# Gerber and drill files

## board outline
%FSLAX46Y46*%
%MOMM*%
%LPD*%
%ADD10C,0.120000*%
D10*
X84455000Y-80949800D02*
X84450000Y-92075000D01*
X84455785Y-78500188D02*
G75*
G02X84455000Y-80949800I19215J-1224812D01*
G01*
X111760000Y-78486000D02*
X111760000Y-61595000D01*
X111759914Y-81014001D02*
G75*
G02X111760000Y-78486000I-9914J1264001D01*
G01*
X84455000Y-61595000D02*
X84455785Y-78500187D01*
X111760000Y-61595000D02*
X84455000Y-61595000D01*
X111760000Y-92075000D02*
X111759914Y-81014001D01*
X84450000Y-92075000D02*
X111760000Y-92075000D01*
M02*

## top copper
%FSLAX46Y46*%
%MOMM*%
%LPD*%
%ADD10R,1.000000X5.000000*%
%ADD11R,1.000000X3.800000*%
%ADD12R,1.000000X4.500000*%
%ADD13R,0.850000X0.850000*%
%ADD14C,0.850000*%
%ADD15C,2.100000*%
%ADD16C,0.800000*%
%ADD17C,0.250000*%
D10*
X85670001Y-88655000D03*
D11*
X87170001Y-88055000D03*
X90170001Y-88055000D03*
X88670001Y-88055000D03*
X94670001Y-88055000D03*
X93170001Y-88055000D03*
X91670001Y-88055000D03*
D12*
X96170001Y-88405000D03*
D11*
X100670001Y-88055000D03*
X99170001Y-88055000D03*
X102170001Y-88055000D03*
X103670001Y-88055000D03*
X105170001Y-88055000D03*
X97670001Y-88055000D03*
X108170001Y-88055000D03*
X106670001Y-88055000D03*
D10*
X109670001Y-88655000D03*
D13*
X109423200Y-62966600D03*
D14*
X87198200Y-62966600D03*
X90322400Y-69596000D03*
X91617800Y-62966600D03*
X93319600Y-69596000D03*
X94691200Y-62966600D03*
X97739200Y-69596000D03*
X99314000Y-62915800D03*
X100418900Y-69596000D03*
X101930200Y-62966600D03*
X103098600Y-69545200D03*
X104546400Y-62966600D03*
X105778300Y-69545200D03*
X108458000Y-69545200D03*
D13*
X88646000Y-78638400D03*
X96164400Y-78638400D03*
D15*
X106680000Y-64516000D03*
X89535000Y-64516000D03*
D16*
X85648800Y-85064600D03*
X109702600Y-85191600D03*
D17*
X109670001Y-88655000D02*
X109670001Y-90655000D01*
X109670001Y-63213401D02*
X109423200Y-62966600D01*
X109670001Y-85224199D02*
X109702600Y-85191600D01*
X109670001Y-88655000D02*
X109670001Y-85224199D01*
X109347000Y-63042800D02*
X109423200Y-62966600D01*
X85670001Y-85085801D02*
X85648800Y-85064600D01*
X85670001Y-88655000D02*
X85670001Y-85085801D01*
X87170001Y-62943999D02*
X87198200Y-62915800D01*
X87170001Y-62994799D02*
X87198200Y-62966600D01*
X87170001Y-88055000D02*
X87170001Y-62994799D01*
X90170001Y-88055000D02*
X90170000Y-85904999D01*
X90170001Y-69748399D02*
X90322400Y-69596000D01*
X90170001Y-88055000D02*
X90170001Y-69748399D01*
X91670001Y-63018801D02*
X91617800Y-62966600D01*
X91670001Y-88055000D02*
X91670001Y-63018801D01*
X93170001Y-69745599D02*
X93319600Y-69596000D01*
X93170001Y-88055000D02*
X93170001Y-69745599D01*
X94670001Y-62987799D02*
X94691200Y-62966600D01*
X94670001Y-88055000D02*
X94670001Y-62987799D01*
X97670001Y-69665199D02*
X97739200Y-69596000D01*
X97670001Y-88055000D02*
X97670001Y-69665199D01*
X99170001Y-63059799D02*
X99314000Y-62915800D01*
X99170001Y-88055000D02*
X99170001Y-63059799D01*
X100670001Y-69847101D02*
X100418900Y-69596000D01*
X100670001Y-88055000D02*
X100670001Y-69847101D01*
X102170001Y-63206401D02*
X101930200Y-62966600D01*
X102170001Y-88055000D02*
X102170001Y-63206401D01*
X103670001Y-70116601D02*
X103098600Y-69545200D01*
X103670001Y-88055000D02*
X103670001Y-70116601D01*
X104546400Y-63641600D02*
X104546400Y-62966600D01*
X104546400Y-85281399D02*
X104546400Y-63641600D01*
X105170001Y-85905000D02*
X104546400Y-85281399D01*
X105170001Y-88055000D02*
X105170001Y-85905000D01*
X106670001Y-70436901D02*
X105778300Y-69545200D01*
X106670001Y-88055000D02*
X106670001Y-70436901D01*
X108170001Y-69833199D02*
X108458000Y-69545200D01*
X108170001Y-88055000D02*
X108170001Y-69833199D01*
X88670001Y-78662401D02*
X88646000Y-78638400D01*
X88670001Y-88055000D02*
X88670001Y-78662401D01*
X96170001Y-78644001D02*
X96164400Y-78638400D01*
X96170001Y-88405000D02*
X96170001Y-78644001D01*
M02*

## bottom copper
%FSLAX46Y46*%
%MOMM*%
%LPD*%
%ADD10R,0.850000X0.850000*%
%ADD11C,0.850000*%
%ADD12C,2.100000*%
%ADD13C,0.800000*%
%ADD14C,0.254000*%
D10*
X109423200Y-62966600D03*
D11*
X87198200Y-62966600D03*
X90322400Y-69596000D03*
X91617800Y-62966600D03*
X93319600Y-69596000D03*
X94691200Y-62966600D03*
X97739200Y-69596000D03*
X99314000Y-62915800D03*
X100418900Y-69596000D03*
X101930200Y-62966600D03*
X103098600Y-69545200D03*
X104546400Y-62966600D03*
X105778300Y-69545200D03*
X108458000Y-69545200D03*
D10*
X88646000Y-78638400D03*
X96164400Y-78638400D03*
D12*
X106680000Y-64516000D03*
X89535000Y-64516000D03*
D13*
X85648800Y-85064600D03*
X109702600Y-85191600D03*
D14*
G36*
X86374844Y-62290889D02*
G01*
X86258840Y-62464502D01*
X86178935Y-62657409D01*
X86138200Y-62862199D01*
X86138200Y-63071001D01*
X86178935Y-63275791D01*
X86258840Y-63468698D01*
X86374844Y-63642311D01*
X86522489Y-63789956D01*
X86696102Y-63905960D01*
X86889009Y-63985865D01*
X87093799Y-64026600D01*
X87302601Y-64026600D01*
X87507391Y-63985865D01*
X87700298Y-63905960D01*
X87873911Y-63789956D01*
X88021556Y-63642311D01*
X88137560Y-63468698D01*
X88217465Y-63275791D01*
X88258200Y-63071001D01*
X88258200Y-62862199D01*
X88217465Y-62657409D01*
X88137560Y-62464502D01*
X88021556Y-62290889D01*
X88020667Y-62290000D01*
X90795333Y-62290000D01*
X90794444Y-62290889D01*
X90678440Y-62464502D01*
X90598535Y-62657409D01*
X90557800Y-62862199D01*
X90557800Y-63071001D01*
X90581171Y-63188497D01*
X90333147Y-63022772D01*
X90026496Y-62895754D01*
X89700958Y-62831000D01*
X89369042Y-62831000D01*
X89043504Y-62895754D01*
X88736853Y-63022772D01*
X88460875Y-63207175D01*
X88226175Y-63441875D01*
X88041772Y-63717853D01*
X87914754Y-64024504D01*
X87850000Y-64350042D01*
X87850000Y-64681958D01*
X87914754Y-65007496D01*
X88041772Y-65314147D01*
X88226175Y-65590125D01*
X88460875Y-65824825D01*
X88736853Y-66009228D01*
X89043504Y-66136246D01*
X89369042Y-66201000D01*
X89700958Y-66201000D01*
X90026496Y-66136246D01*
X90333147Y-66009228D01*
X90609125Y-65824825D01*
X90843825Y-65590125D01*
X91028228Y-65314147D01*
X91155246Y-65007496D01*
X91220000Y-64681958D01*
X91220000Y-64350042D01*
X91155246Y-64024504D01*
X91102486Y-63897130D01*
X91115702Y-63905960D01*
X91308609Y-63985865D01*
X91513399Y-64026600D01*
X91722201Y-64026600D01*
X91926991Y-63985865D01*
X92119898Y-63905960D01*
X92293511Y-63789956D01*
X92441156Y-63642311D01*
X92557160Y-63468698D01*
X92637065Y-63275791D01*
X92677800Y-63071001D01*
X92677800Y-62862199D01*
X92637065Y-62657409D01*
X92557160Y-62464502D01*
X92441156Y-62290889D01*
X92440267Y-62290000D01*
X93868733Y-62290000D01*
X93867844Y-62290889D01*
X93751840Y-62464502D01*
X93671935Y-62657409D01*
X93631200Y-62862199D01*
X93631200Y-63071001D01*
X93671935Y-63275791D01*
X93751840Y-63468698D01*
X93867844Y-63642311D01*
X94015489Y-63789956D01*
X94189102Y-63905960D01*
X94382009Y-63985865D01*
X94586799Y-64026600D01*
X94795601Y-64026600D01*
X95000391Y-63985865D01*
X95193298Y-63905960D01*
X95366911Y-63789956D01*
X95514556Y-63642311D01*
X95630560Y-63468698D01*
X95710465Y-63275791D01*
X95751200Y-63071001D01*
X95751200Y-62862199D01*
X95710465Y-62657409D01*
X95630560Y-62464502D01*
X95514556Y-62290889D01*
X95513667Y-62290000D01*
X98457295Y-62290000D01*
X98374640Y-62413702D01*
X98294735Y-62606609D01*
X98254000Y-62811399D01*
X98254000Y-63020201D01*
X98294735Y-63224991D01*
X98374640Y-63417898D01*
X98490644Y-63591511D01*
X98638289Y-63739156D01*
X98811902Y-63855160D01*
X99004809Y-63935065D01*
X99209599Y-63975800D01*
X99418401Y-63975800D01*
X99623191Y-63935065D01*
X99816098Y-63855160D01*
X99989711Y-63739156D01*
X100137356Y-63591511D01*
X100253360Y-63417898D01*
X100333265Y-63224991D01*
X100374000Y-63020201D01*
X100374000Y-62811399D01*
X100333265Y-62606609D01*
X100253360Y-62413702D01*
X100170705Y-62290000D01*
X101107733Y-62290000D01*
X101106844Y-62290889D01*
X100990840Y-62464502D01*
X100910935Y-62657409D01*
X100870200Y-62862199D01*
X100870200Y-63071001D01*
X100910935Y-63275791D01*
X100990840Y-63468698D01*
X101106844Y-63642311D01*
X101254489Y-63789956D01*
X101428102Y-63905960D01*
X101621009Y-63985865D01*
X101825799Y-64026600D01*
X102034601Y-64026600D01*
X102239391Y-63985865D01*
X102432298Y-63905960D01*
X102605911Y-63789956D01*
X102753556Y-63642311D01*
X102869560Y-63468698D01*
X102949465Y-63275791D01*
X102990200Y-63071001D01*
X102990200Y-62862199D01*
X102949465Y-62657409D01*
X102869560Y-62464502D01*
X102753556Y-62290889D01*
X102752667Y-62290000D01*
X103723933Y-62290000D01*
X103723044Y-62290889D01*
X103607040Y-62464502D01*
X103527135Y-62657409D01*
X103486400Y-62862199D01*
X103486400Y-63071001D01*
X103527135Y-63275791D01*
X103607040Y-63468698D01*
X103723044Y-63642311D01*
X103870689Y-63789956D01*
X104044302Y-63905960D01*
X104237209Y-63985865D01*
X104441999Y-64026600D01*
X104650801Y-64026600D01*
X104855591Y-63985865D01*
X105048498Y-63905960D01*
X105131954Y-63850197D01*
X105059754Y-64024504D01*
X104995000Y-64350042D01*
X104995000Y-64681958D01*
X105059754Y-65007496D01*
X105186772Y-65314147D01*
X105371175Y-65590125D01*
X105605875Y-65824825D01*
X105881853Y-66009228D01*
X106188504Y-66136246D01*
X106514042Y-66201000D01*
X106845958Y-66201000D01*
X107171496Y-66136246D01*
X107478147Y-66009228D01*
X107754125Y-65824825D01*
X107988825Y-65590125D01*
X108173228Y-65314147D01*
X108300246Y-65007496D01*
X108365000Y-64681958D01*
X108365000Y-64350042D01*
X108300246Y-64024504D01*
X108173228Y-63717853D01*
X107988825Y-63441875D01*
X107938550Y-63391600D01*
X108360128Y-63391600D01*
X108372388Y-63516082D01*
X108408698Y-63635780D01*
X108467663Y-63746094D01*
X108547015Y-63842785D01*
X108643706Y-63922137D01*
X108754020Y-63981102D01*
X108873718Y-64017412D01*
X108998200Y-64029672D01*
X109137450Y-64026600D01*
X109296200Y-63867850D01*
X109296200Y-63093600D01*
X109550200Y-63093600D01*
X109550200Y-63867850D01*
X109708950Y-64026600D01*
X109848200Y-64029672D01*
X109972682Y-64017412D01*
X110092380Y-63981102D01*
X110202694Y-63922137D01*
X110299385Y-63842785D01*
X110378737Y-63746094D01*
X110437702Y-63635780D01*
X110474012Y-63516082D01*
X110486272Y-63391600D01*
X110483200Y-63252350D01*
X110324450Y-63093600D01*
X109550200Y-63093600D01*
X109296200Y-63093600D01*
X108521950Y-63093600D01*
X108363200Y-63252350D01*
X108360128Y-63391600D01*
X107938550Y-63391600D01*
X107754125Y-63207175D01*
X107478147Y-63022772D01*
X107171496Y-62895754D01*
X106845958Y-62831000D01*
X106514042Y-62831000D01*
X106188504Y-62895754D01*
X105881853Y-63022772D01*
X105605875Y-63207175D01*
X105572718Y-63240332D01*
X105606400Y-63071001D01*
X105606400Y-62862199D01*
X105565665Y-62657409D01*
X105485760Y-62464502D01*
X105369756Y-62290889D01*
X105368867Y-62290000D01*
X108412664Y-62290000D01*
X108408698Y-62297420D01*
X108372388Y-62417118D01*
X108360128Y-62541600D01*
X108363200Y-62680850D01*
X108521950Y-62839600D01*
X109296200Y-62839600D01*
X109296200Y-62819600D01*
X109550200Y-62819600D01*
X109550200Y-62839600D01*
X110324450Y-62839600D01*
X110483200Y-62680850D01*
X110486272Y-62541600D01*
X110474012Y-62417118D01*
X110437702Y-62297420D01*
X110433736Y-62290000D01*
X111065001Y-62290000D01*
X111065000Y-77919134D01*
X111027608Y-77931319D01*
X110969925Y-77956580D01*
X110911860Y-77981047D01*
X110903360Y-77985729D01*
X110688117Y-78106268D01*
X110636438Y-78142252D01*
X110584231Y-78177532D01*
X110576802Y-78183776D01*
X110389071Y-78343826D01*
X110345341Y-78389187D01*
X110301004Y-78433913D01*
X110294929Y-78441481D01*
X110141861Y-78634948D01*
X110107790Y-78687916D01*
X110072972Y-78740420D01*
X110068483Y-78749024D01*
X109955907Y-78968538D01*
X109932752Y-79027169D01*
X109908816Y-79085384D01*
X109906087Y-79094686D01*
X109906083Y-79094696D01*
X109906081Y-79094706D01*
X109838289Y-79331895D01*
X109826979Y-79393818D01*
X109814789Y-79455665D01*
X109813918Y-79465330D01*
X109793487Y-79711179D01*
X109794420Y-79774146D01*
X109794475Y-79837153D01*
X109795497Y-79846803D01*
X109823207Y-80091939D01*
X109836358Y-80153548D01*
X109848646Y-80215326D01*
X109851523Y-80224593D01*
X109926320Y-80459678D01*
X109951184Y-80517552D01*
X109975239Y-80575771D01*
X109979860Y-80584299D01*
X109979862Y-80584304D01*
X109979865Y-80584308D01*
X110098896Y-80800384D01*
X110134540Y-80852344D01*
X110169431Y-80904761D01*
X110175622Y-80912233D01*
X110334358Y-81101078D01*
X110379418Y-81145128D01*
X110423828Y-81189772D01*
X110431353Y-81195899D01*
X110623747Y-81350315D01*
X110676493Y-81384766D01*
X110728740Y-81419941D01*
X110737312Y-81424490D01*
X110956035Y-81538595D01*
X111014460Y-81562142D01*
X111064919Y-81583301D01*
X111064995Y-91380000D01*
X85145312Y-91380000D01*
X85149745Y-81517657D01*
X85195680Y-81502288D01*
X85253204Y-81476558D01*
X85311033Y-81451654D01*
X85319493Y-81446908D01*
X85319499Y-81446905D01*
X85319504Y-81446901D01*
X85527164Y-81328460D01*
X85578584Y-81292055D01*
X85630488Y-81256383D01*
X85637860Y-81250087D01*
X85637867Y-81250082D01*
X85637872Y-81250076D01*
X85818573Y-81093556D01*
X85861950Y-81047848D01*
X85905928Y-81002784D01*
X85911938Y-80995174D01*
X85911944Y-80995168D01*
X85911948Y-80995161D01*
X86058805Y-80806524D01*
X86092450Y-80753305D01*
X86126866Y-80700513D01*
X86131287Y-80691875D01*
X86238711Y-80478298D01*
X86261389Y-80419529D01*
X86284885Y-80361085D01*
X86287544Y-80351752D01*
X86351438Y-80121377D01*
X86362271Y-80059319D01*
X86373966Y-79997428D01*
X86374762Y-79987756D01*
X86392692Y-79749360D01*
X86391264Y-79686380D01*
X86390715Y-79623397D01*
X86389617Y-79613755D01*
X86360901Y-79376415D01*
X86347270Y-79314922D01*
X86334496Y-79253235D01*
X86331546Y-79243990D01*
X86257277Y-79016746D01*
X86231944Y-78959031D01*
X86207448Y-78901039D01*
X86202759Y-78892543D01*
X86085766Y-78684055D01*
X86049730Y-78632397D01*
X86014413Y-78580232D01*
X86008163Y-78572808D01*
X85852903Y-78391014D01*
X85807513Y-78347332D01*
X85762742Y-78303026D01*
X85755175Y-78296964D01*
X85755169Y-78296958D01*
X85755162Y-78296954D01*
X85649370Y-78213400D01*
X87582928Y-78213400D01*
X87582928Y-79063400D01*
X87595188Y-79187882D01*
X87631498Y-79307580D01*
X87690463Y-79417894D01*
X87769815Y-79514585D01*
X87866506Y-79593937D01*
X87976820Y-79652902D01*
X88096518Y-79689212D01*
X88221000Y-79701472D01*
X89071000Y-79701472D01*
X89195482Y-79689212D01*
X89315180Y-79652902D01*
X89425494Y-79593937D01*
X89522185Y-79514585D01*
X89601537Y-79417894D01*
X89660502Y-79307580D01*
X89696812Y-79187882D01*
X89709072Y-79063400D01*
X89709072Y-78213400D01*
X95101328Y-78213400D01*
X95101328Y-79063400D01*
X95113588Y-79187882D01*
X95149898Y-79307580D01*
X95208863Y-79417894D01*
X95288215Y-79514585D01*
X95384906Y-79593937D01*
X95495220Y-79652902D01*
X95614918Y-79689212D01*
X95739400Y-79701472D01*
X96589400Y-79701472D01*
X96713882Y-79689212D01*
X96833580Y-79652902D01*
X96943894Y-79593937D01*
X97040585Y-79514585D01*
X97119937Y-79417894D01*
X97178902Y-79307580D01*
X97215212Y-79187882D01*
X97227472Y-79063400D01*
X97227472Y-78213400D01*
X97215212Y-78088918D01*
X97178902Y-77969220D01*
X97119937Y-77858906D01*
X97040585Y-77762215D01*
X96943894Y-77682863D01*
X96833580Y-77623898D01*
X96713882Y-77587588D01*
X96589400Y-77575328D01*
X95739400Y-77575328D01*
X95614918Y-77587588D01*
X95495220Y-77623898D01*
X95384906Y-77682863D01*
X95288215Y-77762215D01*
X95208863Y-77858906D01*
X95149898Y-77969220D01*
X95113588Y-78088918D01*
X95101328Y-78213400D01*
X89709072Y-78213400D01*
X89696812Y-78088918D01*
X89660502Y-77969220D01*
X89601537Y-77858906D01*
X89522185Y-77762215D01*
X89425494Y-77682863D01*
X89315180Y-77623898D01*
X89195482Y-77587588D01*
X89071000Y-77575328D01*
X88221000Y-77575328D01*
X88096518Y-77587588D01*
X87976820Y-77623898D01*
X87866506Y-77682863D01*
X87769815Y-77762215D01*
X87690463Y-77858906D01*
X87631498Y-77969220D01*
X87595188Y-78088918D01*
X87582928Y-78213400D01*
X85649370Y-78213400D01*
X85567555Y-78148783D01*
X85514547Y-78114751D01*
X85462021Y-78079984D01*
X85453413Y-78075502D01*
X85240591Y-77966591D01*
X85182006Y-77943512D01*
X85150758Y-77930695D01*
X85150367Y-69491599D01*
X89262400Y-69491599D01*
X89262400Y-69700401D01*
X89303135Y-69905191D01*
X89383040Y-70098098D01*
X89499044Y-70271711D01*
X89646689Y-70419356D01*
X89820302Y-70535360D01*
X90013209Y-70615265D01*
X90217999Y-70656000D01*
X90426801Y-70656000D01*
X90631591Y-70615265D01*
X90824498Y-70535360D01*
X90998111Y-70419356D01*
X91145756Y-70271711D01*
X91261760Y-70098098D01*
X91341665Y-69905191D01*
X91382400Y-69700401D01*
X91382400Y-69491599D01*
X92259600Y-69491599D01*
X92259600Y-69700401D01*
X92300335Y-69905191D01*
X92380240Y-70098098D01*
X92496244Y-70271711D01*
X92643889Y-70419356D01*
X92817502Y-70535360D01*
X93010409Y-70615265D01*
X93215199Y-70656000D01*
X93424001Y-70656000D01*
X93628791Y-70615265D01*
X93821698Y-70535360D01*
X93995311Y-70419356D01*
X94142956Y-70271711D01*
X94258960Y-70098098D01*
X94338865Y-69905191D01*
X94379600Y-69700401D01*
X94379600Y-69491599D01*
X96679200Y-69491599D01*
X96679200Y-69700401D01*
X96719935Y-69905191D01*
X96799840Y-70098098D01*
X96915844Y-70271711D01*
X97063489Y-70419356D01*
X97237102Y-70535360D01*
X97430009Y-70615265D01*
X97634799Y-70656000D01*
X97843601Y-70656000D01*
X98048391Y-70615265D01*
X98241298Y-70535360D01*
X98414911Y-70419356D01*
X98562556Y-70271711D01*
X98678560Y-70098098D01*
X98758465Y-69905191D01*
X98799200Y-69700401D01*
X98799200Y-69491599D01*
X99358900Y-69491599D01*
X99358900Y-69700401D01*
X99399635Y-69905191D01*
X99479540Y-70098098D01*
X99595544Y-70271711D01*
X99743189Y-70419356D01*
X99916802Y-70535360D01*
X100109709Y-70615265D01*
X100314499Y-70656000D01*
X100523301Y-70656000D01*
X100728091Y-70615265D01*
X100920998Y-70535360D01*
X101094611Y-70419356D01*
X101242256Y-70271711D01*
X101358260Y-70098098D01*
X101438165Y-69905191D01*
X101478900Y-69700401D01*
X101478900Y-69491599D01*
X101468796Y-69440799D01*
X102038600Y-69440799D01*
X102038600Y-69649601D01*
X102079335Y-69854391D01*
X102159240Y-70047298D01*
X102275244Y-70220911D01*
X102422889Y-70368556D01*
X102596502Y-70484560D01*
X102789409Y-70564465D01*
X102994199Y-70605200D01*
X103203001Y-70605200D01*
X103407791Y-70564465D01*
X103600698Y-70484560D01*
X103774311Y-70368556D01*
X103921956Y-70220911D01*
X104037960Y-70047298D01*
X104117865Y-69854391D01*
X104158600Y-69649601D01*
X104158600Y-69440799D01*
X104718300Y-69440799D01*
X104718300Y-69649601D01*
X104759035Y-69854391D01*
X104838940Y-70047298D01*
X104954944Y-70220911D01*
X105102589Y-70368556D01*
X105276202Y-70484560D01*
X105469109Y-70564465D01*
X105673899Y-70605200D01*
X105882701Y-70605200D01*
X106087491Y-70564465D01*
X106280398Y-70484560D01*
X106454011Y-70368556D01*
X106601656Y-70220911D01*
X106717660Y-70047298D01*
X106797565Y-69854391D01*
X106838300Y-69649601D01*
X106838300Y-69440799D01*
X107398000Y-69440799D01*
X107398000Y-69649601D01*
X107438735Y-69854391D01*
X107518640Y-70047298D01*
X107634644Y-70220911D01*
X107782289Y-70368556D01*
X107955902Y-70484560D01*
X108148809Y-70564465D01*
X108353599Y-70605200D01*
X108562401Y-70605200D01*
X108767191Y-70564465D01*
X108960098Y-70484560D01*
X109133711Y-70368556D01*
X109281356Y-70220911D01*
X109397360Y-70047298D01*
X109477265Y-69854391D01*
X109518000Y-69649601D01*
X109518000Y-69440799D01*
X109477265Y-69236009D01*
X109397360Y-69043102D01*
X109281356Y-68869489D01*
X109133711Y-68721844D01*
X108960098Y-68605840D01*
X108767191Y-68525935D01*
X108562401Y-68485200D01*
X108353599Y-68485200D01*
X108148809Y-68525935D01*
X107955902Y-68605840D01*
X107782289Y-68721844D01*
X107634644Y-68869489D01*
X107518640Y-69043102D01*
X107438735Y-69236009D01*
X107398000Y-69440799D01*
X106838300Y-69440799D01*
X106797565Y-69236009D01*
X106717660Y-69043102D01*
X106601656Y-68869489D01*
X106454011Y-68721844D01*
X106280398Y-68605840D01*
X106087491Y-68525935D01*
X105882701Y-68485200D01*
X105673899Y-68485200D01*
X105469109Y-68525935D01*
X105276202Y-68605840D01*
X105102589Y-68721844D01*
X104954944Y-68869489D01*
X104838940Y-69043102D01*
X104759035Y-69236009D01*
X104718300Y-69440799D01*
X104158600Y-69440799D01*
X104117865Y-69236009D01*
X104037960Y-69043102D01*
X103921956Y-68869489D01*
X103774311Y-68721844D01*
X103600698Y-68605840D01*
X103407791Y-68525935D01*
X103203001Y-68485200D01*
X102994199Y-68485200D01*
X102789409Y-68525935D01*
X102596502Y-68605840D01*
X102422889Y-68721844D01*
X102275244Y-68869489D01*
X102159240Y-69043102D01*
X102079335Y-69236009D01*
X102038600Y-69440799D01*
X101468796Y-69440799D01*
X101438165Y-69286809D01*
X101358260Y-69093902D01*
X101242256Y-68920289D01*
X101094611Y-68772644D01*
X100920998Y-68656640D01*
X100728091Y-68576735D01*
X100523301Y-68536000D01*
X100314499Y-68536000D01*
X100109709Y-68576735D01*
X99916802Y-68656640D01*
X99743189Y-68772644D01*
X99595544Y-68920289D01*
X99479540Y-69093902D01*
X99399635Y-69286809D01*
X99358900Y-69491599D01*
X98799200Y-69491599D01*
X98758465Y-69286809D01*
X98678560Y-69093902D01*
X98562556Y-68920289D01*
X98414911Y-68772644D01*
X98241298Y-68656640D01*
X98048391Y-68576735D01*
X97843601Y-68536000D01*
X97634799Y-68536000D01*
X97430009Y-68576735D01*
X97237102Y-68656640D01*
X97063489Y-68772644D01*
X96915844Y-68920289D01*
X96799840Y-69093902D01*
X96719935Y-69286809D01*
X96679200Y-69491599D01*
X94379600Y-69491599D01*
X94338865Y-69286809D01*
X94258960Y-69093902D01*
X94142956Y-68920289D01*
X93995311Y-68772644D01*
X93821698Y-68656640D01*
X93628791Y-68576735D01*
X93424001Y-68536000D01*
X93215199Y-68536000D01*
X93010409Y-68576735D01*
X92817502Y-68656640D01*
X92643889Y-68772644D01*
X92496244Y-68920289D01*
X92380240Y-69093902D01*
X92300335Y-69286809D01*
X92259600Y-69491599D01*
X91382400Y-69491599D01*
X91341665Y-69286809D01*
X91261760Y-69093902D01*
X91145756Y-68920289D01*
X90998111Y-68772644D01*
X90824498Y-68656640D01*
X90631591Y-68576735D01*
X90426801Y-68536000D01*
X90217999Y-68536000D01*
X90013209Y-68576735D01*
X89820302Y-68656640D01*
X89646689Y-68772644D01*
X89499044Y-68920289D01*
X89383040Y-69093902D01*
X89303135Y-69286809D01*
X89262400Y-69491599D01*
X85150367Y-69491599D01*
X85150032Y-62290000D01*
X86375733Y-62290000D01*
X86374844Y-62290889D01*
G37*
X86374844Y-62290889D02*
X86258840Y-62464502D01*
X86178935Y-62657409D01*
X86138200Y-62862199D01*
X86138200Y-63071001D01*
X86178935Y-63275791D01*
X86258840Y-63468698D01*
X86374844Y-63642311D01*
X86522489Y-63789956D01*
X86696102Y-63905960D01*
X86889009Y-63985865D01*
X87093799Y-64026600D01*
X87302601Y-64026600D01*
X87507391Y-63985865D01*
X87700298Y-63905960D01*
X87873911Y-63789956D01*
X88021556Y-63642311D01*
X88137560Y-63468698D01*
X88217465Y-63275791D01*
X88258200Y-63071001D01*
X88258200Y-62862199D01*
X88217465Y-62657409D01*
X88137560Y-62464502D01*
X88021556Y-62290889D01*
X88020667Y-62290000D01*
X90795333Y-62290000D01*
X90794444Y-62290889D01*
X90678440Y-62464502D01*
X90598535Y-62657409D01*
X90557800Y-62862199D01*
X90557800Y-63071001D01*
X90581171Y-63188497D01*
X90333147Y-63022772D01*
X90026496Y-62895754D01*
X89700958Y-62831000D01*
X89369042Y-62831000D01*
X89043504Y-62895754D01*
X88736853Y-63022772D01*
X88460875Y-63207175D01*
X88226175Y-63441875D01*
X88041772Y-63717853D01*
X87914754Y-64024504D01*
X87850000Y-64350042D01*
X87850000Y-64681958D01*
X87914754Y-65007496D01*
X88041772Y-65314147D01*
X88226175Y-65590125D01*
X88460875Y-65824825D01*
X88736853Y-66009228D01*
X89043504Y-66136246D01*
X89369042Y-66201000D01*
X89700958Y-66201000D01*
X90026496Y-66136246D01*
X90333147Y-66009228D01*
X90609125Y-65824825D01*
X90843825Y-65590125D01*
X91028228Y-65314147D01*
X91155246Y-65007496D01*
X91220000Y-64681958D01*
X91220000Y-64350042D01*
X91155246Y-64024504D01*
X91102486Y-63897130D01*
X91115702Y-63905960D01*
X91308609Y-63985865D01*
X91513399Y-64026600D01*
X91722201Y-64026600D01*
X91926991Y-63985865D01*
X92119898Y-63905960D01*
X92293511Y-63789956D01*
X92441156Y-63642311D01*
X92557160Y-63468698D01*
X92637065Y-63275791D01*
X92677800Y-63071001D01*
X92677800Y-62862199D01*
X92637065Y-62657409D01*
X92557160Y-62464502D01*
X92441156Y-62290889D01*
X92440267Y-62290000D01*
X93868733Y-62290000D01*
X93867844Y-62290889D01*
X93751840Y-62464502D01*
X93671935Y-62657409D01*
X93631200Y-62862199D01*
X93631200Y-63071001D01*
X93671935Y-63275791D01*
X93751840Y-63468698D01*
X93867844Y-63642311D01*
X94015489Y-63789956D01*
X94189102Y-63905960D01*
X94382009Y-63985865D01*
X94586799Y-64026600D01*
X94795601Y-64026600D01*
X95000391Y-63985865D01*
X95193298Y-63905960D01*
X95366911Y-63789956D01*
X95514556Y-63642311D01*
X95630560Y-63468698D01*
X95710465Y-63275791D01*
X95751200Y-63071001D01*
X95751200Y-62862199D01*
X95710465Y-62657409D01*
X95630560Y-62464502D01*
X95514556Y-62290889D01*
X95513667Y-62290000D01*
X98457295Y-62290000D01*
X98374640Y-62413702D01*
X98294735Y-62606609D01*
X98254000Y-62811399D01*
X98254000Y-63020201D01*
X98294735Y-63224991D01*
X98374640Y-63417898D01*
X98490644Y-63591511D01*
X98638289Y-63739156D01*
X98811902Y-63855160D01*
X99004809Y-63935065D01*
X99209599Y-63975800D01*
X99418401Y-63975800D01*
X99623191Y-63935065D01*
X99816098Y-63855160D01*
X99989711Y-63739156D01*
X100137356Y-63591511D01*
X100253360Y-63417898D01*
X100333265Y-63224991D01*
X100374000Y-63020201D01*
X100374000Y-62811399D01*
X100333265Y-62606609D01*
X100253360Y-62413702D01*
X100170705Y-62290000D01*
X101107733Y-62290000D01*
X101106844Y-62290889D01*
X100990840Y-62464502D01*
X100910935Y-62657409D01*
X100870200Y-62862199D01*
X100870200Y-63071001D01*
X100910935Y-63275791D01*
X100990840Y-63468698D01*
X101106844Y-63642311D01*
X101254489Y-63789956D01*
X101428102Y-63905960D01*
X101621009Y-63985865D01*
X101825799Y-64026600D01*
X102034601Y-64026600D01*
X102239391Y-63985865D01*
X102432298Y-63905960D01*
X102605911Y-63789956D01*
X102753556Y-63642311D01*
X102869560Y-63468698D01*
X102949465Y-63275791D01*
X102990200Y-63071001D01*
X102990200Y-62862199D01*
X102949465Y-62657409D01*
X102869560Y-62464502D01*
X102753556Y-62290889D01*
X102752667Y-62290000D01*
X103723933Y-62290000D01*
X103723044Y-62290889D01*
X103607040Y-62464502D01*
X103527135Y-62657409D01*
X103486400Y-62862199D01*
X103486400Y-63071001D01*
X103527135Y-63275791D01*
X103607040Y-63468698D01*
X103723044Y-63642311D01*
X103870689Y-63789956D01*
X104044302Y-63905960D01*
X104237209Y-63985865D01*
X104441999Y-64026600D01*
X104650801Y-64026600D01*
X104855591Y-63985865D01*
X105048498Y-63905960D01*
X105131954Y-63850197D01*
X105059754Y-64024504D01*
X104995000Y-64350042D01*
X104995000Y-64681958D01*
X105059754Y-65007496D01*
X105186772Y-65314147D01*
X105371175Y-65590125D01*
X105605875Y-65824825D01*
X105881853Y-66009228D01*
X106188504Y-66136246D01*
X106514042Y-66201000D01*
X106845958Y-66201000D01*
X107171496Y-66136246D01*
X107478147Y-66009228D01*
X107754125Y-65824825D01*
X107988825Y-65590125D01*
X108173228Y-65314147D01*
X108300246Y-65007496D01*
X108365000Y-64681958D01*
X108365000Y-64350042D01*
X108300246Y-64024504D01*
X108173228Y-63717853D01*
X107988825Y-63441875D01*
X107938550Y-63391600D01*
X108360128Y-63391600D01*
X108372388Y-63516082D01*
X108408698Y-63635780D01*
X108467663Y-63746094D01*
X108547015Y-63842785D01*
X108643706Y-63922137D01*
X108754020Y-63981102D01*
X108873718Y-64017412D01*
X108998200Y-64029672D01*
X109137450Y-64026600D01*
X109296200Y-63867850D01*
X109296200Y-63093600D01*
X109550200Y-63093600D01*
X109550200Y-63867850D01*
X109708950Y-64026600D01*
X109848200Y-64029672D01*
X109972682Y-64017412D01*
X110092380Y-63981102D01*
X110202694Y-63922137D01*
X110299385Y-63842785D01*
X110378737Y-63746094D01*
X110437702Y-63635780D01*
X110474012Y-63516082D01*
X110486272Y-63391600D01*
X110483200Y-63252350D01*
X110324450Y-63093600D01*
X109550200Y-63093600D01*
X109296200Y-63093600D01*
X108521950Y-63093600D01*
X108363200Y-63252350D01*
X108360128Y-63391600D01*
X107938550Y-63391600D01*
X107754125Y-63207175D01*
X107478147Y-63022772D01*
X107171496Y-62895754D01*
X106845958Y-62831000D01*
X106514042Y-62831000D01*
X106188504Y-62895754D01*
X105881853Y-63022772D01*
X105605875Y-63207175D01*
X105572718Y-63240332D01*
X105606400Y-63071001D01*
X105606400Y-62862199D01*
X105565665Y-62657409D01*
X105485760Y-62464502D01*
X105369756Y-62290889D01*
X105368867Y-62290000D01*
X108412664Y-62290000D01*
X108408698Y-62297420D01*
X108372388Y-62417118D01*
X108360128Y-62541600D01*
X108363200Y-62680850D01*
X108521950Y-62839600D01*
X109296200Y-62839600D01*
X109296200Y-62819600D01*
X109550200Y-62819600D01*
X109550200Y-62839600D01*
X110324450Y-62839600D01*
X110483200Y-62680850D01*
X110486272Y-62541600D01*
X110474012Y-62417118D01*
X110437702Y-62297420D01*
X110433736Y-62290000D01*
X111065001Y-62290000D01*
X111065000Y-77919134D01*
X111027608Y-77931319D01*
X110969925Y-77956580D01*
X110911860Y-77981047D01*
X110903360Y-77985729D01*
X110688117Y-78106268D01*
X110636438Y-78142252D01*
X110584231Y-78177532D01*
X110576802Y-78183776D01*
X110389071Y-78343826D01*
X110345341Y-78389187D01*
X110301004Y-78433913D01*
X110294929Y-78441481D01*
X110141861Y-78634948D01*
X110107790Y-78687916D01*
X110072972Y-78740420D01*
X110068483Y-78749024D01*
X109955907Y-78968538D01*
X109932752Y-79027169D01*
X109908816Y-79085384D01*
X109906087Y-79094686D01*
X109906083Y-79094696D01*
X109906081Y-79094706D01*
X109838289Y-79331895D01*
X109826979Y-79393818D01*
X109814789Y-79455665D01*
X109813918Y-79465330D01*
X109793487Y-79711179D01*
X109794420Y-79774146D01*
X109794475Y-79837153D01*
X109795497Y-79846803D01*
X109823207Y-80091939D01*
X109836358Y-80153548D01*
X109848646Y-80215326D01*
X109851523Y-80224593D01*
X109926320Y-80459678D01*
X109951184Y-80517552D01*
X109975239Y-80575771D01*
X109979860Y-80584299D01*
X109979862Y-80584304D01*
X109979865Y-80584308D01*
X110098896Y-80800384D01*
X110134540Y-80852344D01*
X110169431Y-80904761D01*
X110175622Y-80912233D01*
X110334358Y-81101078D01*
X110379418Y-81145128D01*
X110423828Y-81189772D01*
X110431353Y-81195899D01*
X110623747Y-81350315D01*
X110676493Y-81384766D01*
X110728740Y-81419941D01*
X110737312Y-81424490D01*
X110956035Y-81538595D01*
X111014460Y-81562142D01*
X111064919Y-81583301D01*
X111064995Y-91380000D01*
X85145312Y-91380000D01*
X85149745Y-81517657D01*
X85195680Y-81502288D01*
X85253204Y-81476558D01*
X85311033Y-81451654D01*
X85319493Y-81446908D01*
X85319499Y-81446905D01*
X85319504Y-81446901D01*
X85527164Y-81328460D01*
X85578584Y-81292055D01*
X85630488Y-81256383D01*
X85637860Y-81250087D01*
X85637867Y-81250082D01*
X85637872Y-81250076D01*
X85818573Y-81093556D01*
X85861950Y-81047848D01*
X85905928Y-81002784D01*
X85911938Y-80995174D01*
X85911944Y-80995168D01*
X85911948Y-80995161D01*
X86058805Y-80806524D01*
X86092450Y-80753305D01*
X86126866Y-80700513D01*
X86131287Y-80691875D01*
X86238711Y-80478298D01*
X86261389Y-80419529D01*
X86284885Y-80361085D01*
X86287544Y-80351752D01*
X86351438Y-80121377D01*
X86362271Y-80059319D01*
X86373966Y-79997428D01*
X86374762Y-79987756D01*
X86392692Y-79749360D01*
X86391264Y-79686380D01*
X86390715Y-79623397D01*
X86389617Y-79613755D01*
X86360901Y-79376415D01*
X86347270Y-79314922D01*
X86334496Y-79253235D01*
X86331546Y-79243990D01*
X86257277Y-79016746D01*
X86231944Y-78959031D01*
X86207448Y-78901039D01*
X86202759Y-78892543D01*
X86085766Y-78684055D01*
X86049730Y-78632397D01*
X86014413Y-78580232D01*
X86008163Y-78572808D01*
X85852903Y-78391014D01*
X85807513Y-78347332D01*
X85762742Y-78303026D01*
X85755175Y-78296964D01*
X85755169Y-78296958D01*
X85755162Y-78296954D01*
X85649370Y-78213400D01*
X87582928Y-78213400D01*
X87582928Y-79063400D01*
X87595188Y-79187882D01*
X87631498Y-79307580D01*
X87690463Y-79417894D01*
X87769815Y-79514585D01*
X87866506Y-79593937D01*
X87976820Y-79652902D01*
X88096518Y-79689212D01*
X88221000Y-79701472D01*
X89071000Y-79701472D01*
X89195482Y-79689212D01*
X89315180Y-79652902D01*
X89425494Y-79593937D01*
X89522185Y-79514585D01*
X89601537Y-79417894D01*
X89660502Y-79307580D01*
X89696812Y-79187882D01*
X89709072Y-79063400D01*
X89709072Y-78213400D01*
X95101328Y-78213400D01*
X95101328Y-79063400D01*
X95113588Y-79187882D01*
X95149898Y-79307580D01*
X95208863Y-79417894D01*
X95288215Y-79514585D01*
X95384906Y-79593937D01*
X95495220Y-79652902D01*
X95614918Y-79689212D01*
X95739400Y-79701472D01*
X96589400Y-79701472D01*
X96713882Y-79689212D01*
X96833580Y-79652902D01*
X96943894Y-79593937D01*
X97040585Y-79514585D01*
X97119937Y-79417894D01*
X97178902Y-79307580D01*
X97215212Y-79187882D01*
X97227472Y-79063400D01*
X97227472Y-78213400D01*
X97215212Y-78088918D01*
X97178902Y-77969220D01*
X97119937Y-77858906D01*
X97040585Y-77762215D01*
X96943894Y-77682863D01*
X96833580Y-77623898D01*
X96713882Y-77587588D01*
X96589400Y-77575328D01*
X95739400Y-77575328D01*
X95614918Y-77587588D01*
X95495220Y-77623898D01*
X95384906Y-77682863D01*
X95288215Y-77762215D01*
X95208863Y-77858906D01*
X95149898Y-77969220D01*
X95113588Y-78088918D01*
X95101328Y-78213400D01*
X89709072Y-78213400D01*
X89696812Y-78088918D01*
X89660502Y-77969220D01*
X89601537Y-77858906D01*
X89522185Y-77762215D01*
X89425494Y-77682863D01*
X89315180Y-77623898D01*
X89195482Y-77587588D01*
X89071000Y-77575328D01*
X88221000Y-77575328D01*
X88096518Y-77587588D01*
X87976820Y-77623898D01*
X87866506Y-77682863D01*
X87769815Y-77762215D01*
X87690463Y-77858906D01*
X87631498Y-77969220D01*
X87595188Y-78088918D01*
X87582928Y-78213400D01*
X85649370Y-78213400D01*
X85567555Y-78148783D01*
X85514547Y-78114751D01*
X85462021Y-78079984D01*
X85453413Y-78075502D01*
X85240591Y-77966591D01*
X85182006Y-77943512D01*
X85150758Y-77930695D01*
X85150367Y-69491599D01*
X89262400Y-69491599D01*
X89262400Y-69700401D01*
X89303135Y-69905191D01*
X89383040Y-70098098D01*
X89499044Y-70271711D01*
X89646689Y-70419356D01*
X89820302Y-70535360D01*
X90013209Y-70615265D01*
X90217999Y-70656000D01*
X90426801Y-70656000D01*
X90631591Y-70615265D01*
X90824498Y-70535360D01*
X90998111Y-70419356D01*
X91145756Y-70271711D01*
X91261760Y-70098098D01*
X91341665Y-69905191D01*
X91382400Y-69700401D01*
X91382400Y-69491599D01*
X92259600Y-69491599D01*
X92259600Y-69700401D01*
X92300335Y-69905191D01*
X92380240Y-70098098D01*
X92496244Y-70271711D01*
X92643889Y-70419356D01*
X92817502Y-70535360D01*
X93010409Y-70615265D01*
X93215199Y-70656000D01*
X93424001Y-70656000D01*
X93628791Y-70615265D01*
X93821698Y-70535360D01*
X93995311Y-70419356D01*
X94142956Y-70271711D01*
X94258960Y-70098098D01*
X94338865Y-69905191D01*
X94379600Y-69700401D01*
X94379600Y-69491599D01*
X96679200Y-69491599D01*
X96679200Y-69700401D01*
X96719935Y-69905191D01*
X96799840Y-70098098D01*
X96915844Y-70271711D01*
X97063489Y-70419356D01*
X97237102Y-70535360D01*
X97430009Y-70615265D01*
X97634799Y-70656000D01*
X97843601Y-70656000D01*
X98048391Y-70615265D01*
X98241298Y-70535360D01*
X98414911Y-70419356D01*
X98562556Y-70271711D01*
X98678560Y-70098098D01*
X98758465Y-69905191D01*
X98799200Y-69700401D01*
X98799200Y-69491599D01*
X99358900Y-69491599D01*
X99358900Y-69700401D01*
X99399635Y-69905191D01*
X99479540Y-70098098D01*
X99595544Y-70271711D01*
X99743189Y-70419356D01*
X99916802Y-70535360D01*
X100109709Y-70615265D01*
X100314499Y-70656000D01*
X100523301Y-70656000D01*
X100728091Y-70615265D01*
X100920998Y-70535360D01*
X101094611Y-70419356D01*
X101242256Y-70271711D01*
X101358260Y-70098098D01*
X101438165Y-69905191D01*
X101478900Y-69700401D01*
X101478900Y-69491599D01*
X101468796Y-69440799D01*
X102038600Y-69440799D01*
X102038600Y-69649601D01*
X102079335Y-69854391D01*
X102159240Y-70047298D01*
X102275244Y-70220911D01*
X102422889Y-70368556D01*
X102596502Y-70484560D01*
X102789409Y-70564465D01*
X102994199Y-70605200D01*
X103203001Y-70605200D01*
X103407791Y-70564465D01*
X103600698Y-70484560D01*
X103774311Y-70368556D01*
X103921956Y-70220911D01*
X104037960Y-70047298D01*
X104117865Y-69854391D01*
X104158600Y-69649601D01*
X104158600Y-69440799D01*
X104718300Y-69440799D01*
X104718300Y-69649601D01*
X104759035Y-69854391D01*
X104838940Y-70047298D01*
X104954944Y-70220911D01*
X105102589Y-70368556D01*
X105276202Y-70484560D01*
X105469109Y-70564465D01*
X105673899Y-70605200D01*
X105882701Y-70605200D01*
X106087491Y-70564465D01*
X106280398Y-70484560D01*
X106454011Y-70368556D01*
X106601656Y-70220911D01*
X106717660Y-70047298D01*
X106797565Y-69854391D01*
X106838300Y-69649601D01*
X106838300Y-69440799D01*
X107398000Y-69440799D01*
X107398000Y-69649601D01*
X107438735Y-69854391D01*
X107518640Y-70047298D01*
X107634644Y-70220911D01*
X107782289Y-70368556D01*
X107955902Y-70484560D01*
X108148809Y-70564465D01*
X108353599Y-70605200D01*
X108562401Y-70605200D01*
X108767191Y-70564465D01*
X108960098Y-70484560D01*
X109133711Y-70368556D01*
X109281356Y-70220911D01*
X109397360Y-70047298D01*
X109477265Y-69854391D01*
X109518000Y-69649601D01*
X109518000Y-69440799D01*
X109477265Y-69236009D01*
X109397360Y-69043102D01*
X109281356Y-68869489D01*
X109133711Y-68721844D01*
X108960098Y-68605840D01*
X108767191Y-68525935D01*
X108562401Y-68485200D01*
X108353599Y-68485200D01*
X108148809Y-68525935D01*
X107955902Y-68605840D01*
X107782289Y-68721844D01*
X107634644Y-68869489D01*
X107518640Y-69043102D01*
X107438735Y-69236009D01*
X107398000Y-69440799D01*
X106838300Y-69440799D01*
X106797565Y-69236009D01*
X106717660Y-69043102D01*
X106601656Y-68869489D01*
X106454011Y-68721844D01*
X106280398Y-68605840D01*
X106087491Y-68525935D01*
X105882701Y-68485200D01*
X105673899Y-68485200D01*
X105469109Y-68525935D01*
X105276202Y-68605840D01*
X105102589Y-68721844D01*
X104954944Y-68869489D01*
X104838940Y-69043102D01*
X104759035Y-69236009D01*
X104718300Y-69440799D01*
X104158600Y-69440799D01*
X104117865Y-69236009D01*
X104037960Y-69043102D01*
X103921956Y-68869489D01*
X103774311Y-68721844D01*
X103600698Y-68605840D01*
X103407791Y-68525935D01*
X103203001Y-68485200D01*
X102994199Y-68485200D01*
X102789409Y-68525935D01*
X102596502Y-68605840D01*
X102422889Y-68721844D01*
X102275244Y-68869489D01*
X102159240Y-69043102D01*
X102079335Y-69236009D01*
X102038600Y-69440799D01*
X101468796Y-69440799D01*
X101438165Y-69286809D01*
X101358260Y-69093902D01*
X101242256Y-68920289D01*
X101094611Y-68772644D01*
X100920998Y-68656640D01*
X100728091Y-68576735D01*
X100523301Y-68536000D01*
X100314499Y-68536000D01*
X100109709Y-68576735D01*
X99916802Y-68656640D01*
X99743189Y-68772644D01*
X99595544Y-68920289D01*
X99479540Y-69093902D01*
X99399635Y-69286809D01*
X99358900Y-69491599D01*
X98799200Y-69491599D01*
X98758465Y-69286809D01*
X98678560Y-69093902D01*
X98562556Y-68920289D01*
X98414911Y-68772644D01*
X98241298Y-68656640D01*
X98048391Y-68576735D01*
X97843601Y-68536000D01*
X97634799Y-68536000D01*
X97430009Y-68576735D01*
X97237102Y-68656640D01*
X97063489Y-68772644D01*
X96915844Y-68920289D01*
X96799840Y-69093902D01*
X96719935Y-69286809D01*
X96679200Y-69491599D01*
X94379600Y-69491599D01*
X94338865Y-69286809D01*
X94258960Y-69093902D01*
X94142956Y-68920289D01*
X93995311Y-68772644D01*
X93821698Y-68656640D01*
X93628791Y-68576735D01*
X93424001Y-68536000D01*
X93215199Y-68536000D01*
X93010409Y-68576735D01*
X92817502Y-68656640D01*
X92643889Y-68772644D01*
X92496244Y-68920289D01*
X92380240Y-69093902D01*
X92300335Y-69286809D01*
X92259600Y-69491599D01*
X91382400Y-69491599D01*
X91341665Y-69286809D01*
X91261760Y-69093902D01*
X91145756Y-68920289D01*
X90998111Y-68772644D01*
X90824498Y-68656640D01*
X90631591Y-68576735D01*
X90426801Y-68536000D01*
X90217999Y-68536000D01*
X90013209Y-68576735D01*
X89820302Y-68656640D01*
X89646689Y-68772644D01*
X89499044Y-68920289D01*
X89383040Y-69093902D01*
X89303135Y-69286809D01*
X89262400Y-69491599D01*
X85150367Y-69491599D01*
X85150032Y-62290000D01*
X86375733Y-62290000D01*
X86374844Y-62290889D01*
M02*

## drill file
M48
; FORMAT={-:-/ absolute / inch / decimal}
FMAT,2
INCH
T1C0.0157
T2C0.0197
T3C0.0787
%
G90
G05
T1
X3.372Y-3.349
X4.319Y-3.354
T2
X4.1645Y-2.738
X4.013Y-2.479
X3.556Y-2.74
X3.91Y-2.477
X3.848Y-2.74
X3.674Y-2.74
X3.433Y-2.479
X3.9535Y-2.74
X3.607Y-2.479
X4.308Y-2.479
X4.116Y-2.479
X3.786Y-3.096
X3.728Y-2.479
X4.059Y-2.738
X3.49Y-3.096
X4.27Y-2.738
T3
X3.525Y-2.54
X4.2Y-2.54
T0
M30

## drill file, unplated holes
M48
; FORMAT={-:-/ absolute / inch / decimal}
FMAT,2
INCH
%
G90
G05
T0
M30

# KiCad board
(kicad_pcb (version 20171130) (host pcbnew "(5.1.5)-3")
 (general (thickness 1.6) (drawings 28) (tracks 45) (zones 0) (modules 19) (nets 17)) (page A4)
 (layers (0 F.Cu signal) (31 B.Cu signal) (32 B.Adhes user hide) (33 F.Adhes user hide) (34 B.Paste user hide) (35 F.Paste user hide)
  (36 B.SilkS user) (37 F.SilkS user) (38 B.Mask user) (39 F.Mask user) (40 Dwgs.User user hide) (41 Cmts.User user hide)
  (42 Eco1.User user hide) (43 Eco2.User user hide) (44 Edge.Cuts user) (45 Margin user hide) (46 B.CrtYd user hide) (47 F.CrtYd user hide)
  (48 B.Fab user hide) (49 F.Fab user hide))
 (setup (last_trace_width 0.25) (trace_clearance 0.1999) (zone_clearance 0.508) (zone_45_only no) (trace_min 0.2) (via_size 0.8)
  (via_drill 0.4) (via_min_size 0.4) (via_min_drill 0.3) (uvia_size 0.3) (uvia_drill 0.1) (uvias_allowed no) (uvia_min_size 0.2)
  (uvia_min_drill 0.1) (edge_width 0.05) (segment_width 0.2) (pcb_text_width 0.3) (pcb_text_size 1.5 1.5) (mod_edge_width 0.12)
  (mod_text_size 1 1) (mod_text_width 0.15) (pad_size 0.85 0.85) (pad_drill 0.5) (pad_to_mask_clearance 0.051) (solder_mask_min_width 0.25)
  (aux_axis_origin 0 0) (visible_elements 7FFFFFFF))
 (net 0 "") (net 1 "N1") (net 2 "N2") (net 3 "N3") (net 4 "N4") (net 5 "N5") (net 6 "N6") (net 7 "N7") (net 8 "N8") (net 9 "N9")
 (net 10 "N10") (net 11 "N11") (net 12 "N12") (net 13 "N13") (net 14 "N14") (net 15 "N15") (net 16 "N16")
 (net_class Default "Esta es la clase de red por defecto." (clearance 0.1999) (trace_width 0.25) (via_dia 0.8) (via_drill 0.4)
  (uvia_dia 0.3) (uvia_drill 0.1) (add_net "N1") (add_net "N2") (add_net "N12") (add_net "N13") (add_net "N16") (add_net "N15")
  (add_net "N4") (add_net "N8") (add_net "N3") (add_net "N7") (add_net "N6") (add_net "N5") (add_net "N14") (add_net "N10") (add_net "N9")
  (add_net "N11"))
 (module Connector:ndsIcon (layer F.Cu) (at 103.4542 85.9536)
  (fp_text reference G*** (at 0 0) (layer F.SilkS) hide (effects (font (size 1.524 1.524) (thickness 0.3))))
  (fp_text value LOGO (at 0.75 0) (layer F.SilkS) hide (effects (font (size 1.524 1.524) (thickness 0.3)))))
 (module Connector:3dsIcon (layer F.Cu) (at 92.2528 86.1314)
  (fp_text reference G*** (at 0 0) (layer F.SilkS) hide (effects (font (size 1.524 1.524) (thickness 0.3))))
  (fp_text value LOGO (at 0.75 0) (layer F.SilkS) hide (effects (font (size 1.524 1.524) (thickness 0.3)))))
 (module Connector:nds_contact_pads (layer F.Cu) (at 92.770001 84.705)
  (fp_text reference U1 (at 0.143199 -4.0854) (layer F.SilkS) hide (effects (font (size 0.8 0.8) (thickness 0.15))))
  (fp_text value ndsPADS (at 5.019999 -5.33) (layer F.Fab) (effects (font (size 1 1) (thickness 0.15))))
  (pad 1 smd rect (at -7.1 3.95) (size 1 5) (layers F.Cu F.Paste F.Mask) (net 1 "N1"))
  (pad 2 smd rect (at -5.6 3.35) (size 1 3.8) (layers F.Cu F.Paste F.Mask) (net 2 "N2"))
  (pad 4 smd rect (at -2.6 3.35) (size 1 3.8) (layers F.Cu F.Paste F.Mask) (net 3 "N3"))
  (pad 3 smd rect (at -4.1 3.35) (size 1 3.8) (layers F.Cu F.Paste F.Mask) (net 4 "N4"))
  (pad 7 smd rect (at 1.9 3.35) (size 1 3.8) (layers F.Cu F.Paste F.Mask) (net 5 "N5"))
  (pad 6 smd rect (at 0.4 3.35) (size 1 3.8) (layers F.Cu F.Paste F.Mask) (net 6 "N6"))
  (pad 5 smd rect (at -1.1 3.35) (size 1 3.8) (layers F.Cu F.Paste F.Mask) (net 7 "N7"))
  (pad 8 smd rect (at 3.4 3.7) (size 1 4.5) (layers F.Cu F.Paste F.Mask) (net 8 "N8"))
  (pad 11 smd rect (at 7.9 3.35) (size 1 3.8) (layers F.Cu F.Paste F.Mask) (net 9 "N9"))
  (pad 10 smd rect (at 6.4 3.35) (size 1 3.8) (layers F.Cu F.Paste F.Mask) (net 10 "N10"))
  (pad 12 smd rect (at 9.4 3.35) (size 1 3.8) (layers F.Cu F.Paste F.Mask) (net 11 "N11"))
  (pad 13 smd rect (at 10.9 3.35) (size 1 3.8) (layers F.Cu F.Paste F.Mask) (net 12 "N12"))
  (pad 14 smd rect (at 12.4 3.35) (size 1 3.8) (layers F.Cu F.Paste F.Mask) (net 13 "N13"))
  (pad 9 smd rect (at 4.9 3.35) (size 1 3.8) (layers F.Cu F.Paste F.Mask) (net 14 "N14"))
  (pad 16 smd rect (at 15.4 3.35) (size 1 3.8) (layers F.Cu F.Paste F.Mask) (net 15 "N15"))
  (pad 15 smd rect (at 13.9 3.35) (size 1 3.8) (layers F.Cu F.Paste F.Mask) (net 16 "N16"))
  (pad 17 smd rect (at 16.9 3.95) (size 1 5) (layers F.Cu F.Paste F.Mask) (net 1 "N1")))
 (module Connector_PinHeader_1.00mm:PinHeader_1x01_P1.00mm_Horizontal (layer F.Cu) (at 109.4232 62.9666 90)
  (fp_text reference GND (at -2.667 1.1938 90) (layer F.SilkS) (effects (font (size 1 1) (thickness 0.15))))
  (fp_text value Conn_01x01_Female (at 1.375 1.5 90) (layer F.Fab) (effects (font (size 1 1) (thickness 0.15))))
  (pad 1 thru_hole rect (at 0 0 90) (size 0.85 0.85) (drill 0.5) (layers *.Cu *.Mask) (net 1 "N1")))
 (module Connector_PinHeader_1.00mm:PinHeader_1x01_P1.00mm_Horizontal (layer F.Cu) (at 87.1982 62.9666 90)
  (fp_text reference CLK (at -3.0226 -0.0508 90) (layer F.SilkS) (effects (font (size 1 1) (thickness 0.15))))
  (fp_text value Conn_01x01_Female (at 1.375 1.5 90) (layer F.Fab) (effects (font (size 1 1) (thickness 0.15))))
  (pad 1 thru_hole circle (at 0 0 90) (size 0.85 0.85) (drill 0.5) (layers *.Cu *.Mask) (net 2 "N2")))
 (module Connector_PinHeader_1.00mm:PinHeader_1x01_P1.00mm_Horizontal (layer F.Cu) (at 90.3224 69.596 90)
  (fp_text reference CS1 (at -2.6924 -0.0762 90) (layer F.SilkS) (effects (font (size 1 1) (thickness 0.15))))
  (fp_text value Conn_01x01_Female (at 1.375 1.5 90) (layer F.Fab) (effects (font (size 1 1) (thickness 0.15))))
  (pad 1 thru_hole circle (at 0 0 90) (size 0.85 0.85) (drill 0.5) (layers *.Cu *.Mask) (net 3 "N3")))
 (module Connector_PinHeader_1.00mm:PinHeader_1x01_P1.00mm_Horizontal (layer F.Cu) (at 91.6178 62.9666 90)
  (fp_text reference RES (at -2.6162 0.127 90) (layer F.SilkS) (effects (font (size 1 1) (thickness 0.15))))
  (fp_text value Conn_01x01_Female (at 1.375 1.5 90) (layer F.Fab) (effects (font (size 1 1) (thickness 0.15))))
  (pad 1 thru_hole circle (at 0 0 90) (size 0.85 0.85) (drill 0.5) (layers *.Cu *.Mask) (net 7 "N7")))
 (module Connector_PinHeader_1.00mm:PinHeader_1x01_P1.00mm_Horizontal (layer F.Cu) (at 93.3196 69.596 90)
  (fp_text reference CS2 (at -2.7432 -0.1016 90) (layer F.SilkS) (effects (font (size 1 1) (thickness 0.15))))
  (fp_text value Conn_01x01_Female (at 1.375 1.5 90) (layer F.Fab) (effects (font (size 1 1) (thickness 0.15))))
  (pad 1 thru_hole circle (at 0 0 90) (size 0.85 0.85) (drill 0.5) (layers *.Cu *.Mask) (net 6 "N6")))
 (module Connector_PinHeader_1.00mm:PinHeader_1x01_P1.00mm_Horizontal (layer F.Cu) (at 94.6912 62.9666 90)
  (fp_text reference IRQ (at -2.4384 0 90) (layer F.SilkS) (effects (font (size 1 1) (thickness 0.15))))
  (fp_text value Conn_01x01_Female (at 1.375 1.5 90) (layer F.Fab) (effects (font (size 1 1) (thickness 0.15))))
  (pad 1 thru_hole circle (at 0 0 90) (size 0.85 0.85) (drill 0.5) (layers *.Cu *.Mask) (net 5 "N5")))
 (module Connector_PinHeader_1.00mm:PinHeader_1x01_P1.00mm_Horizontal (layer F.Cu) (at 97.7392 69.596 90)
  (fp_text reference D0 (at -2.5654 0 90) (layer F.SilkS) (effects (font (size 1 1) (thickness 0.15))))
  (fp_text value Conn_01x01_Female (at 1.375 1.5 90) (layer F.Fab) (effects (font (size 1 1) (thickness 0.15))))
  (pad 1 thru_hole circle (at 0 0 90) (size 0.85 0.85) (drill 0.5) (layers *.Cu *.Mask) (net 14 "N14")))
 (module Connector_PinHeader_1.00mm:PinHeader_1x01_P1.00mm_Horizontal (layer F.Cu) (at 99.314 62.9158 90)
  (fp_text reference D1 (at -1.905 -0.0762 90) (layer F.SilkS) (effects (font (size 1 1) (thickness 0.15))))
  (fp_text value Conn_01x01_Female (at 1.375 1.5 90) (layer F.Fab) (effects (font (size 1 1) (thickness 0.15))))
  (pad 1 thru_hole circle (at 0 0 90) (size 0.85 0.85) (drill 0.5) (layers *.Cu *.Mask) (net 10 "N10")))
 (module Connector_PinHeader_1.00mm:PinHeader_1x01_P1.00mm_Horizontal (layer F.Cu) (at 100.4189 69.596 90)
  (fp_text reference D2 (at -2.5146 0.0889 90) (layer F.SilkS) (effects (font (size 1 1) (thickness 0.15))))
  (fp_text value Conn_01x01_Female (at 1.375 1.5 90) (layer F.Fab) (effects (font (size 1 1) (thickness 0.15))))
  (pad 1 thru_hole circle (at 0 0 90) (size 0.85 0.85) (drill 0.5) (layers *.Cu *.Mask) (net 9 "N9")))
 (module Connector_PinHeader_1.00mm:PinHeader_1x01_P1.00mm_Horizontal (layer F.Cu) (at 101.9302 62.9666 90)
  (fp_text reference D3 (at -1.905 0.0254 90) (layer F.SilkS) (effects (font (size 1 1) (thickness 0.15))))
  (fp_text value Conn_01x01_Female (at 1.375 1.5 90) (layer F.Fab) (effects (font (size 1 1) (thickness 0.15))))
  (pad 1 thru_hole circle (at 0 0 90) (size 0.85 0.85) (drill 0.5) (layers *.Cu *.Mask) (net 11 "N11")))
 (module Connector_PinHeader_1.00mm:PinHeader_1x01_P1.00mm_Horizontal (layer F.Cu) (at 103.0986 69.5452 90)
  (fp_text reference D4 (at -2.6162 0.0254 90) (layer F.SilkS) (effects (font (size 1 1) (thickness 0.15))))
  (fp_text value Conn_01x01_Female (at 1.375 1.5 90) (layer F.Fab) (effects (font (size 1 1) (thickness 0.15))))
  (pad 1 thru_hole circle (at 0 0 90) (size 0.85 0.85) (drill 0.5) (layers *.Cu *.Mask) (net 12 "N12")))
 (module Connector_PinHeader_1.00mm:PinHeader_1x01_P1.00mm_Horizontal (layer F.Cu) (at 104.5464 62.9666 90)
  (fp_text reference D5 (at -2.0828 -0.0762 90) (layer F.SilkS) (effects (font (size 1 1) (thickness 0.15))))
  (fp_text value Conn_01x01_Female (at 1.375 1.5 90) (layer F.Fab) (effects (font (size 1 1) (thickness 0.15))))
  (pad 1 thru_hole circle (at 0 0 90) (size 0.85 0.85) (drill 0.5) (layers *.Cu *.Mask) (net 13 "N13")))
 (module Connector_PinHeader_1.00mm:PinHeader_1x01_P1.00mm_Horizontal (layer F.Cu) (at 105.7783 69.5452 90)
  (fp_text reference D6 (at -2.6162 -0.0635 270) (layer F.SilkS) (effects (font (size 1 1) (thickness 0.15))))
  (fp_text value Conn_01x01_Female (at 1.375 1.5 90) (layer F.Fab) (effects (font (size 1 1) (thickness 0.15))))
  (pad 1 thru_hole circle (at 0 0 90) (size 0.85 0.85) (drill 0.5) (layers *.Cu *.Mask) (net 16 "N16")))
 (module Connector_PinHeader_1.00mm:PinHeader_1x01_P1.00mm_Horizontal (layer F.Cu) (at 108.458 69.5452 90)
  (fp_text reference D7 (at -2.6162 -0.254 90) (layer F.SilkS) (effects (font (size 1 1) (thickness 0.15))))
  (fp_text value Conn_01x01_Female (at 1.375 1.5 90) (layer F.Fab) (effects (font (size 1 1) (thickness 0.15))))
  (pad 1 thru_hole circle (at 0 0 90) (size 0.85 0.85) (drill 0.5) (layers *.Cu *.Mask) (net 15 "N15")))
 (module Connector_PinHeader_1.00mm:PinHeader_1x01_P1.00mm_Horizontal (layer F.Cu) (at 88.646 78.6384 90)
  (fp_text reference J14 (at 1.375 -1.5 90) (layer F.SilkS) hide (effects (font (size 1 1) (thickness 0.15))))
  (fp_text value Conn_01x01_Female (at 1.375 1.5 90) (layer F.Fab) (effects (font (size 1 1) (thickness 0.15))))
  (pad 1 thru_hole rect (at 0 0 90) (size 0.85 0.85) (drill 0.5) (layers *.Cu *.Mask) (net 4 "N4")))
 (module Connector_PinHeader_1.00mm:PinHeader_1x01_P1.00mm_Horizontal (layer F.Cu) (at 96.1644 78.6384 90)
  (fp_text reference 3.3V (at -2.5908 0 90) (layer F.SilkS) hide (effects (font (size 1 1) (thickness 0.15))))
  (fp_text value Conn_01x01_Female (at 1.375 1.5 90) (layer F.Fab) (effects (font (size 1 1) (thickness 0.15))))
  (pad 1 thru_hole rect (at 0 0 90) (size 0.85 0.85) (drill 0.5) (layers *.Cu *.Mask) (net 8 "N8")))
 (gr_line (start 84.455 80.9498) (end 84.45 92.075) (layer Edge.Cuts) (width 0.12))
 (gr_arc (start 84.475 79.725) (end 84.455 80.9498) (angle -181.8343179) (layer Edge.Cuts) (width 0.12))
 (gr_line (start 111.76 78.486) (end 111.76 61.595) (layer Edge.Cuts) (width 0.12))
 (gr_arc (start 111.75 79.75) (end 111.76 78.486) (angle -180.9026615) (layer Edge.Cuts) (width 0.12))
 (gr_line (start 84.455 61.595) (end 84.455785 78.500187) (layer Edge.Cuts) (width 0.12))
 (gr_line (start 111.76 61.595) (end 84.455 61.595) (layer Edge.Cuts) (width 0.12))
 (gr_line (start 111.76 92.075) (end 111.759914 81.014001) (layer Edge.Cuts) (width 0.12))
 (gr_line (start 84.45 92.075) (end 111.76 92.075) (layer Edge.Cuts) (width 0.12))
 (via (at 106.68 64.516) (size 2.1) (drill 2) (layers F.Cu B.Cu) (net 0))
 (via (at 89.535 64.516) (size 2.1) (drill 2) (layers F.Cu B.Cu) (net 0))
 (segment (start 109.670001 88.655) (end 109.670001 90.655) (width 0.25) (layer F.Cu) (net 1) (status 30))
 (segment (start 109.670001 63.213401) (end 109.4232 62.9666) (width 0.25) (layer F.Cu) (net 1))
 (via (at 85.6488 85.0646) (size 0.8) (drill 0.4) (layers F.Cu B.Cu) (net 1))
 (via (at 109.7026 85.1916) (size 0.8) (drill 0.4) (layers F.Cu B.Cu) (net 1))
 (segment (start 109.670001 85.224199) (end 109.7026 85.1916) (width 0.25) (layer F.Cu) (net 1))
 (segment (start 109.670001 88.655) (end 109.670001 85.224199) (width 0.25) (layer F.Cu) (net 1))
 (segment (start 109.347 63.0428) (end 109.4232 62.9666) (width 0.25) (layer F.Cu) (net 1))
 (segment (start 85.670001 85.085801) (end 85.6488 85.0646) (width 0.25) (layer F.Cu) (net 1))
 (segment (start 85.670001 88.655) (end 85.670001 85.085801) (width 0.25) (layer F.Cu) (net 1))
 (segment (start 87.170001 62.943999) (end 87.1982 62.9158) (width 0.25) (layer F.Cu) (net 2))
 (segment (start 87.170001 62.994799) (end 87.1982 62.9666) (width 0.25) (layer F.Cu) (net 2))
 (segment (start 87.170001 88.055) (end 87.170001 62.994799) (width 0.25) (layer F.Cu) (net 2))
 (segment (start 90.170001 88.055) (end 90.17 85.904999) (width 0.25) (layer F.Cu) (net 3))
 (segment (start 90.170001 69.748399) (end 90.3224 69.596) (width 0.25) (layer F.Cu) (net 3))
 (segment (start 90.170001 88.055) (end 90.170001 69.748399) (width 0.25) (layer F.Cu) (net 3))
 (segment (start 91.670001 63.018801) (end 91.6178 62.9666) (width 0.25) (layer F.Cu) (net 7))
 (segment (start 91.670001 88.055) (end 91.670001 63.018801) (width 0.25) (layer F.Cu) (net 7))
 (segment (start 93.170001 69.745599) (end 93.3196 69.596) (width 0.25) (layer F.Cu) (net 6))
 (segment (start 93.170001 88.055) (end 93.170001 69.745599) (width 0.25) (layer F.Cu) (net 6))
 (segment (start 94.670001 62.987799) (end 94.6912 62.9666) (width 0.25) (layer F.Cu) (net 5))
 (segment (start 94.670001 88.055) (end 94.670001 62.987799) (width 0.25) (layer F.Cu) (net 5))
 (segment (start 97.670001 69.665199) (end 97.7392 69.596) (width 0.25) (layer F.Cu) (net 14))
 (segment (start 97.670001 88.055) (end 97.670001 69.665199) (width 0.25) (layer F.Cu) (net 14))
 (segment (start 99.170001 63.059799) (end 99.314 62.9158) (width 0.25) (layer F.Cu) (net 10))
 (segment (start 99.170001 88.055) (end 99.170001 63.059799) (width 0.25) (layer F.Cu) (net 10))
 (segment (start 100.670001 69.847101) (end 100.4189 69.596) (width 0.25) (layer F.Cu) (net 9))
 (segment (start 100.670001 88.055) (end 100.670001 69.847101) (width 0.25) (layer F.Cu) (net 9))
 (segment (start 102.170001 63.206401) (end 101.9302 62.9666) (width 0.25) (layer F.Cu) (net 11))
 (segment (start 102.170001 88.055) (end 102.170001 63.206401) (width 0.25) (layer F.Cu) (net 11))
 (segment (start 103.670001 70.116601) (end 103.0986 69.5452) (width 0.25) (layer F.Cu) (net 12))
 (segment (start 103.670001 88.055) (end 103.670001 70.116601) (width 0.25) (layer F.Cu) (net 12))
 (segment (start 104.5464 63.6416) (end 104.5464 62.9666) (width 0.25) (layer F.Cu) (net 13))
 (segment (start 104.5464 85.281399) (end 104.5464 63.6416) (width 0.25) (layer F.Cu) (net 13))
 (segment (start 105.170001 85.905) (end 104.5464 85.281399) (width 0.25) (layer F.Cu) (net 13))
 (segment (start 105.170001 88.055) (end 105.170001 85.905) (width 0.25) (layer F.Cu) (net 13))
 (segment (start 106.670001 70.436901) (end 105.7783 69.5452) (width 0.25) (layer F.Cu) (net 16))
 (segment (start 106.670001 88.055) (end 106.670001 70.436901) (width 0.25) (layer F.Cu) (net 16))
 (segment (start 108.170001 69.833199) (end 108.458 69.5452) (width 0.25) (layer F.Cu) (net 15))
 (segment (start 108.170001 88.055) (end 108.170001 69.833199) (width 0.25) (layer F.Cu) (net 15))
 (segment (start 88.670001 78.662401) (end 88.646 78.6384) (width 0.25) (layer F.Cu) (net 4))
 (segment (start 88.670001 88.055) (end 88.670001 78.662401) (width 0.25) (layer F.Cu) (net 4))
 (segment (start 96.170001 78.644001) (end 96.1644 78.6384) (width 0.25) (layer F.Cu) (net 8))
 (segment (start 96.170001 88.405) (end 96.170001 78.644001) (width 0.25) (layer F.Cu) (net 8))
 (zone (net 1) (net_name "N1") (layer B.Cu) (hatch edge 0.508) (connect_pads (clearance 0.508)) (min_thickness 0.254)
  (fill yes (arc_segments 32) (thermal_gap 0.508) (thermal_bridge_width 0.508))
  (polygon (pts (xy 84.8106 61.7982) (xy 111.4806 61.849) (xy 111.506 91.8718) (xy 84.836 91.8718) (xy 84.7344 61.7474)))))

